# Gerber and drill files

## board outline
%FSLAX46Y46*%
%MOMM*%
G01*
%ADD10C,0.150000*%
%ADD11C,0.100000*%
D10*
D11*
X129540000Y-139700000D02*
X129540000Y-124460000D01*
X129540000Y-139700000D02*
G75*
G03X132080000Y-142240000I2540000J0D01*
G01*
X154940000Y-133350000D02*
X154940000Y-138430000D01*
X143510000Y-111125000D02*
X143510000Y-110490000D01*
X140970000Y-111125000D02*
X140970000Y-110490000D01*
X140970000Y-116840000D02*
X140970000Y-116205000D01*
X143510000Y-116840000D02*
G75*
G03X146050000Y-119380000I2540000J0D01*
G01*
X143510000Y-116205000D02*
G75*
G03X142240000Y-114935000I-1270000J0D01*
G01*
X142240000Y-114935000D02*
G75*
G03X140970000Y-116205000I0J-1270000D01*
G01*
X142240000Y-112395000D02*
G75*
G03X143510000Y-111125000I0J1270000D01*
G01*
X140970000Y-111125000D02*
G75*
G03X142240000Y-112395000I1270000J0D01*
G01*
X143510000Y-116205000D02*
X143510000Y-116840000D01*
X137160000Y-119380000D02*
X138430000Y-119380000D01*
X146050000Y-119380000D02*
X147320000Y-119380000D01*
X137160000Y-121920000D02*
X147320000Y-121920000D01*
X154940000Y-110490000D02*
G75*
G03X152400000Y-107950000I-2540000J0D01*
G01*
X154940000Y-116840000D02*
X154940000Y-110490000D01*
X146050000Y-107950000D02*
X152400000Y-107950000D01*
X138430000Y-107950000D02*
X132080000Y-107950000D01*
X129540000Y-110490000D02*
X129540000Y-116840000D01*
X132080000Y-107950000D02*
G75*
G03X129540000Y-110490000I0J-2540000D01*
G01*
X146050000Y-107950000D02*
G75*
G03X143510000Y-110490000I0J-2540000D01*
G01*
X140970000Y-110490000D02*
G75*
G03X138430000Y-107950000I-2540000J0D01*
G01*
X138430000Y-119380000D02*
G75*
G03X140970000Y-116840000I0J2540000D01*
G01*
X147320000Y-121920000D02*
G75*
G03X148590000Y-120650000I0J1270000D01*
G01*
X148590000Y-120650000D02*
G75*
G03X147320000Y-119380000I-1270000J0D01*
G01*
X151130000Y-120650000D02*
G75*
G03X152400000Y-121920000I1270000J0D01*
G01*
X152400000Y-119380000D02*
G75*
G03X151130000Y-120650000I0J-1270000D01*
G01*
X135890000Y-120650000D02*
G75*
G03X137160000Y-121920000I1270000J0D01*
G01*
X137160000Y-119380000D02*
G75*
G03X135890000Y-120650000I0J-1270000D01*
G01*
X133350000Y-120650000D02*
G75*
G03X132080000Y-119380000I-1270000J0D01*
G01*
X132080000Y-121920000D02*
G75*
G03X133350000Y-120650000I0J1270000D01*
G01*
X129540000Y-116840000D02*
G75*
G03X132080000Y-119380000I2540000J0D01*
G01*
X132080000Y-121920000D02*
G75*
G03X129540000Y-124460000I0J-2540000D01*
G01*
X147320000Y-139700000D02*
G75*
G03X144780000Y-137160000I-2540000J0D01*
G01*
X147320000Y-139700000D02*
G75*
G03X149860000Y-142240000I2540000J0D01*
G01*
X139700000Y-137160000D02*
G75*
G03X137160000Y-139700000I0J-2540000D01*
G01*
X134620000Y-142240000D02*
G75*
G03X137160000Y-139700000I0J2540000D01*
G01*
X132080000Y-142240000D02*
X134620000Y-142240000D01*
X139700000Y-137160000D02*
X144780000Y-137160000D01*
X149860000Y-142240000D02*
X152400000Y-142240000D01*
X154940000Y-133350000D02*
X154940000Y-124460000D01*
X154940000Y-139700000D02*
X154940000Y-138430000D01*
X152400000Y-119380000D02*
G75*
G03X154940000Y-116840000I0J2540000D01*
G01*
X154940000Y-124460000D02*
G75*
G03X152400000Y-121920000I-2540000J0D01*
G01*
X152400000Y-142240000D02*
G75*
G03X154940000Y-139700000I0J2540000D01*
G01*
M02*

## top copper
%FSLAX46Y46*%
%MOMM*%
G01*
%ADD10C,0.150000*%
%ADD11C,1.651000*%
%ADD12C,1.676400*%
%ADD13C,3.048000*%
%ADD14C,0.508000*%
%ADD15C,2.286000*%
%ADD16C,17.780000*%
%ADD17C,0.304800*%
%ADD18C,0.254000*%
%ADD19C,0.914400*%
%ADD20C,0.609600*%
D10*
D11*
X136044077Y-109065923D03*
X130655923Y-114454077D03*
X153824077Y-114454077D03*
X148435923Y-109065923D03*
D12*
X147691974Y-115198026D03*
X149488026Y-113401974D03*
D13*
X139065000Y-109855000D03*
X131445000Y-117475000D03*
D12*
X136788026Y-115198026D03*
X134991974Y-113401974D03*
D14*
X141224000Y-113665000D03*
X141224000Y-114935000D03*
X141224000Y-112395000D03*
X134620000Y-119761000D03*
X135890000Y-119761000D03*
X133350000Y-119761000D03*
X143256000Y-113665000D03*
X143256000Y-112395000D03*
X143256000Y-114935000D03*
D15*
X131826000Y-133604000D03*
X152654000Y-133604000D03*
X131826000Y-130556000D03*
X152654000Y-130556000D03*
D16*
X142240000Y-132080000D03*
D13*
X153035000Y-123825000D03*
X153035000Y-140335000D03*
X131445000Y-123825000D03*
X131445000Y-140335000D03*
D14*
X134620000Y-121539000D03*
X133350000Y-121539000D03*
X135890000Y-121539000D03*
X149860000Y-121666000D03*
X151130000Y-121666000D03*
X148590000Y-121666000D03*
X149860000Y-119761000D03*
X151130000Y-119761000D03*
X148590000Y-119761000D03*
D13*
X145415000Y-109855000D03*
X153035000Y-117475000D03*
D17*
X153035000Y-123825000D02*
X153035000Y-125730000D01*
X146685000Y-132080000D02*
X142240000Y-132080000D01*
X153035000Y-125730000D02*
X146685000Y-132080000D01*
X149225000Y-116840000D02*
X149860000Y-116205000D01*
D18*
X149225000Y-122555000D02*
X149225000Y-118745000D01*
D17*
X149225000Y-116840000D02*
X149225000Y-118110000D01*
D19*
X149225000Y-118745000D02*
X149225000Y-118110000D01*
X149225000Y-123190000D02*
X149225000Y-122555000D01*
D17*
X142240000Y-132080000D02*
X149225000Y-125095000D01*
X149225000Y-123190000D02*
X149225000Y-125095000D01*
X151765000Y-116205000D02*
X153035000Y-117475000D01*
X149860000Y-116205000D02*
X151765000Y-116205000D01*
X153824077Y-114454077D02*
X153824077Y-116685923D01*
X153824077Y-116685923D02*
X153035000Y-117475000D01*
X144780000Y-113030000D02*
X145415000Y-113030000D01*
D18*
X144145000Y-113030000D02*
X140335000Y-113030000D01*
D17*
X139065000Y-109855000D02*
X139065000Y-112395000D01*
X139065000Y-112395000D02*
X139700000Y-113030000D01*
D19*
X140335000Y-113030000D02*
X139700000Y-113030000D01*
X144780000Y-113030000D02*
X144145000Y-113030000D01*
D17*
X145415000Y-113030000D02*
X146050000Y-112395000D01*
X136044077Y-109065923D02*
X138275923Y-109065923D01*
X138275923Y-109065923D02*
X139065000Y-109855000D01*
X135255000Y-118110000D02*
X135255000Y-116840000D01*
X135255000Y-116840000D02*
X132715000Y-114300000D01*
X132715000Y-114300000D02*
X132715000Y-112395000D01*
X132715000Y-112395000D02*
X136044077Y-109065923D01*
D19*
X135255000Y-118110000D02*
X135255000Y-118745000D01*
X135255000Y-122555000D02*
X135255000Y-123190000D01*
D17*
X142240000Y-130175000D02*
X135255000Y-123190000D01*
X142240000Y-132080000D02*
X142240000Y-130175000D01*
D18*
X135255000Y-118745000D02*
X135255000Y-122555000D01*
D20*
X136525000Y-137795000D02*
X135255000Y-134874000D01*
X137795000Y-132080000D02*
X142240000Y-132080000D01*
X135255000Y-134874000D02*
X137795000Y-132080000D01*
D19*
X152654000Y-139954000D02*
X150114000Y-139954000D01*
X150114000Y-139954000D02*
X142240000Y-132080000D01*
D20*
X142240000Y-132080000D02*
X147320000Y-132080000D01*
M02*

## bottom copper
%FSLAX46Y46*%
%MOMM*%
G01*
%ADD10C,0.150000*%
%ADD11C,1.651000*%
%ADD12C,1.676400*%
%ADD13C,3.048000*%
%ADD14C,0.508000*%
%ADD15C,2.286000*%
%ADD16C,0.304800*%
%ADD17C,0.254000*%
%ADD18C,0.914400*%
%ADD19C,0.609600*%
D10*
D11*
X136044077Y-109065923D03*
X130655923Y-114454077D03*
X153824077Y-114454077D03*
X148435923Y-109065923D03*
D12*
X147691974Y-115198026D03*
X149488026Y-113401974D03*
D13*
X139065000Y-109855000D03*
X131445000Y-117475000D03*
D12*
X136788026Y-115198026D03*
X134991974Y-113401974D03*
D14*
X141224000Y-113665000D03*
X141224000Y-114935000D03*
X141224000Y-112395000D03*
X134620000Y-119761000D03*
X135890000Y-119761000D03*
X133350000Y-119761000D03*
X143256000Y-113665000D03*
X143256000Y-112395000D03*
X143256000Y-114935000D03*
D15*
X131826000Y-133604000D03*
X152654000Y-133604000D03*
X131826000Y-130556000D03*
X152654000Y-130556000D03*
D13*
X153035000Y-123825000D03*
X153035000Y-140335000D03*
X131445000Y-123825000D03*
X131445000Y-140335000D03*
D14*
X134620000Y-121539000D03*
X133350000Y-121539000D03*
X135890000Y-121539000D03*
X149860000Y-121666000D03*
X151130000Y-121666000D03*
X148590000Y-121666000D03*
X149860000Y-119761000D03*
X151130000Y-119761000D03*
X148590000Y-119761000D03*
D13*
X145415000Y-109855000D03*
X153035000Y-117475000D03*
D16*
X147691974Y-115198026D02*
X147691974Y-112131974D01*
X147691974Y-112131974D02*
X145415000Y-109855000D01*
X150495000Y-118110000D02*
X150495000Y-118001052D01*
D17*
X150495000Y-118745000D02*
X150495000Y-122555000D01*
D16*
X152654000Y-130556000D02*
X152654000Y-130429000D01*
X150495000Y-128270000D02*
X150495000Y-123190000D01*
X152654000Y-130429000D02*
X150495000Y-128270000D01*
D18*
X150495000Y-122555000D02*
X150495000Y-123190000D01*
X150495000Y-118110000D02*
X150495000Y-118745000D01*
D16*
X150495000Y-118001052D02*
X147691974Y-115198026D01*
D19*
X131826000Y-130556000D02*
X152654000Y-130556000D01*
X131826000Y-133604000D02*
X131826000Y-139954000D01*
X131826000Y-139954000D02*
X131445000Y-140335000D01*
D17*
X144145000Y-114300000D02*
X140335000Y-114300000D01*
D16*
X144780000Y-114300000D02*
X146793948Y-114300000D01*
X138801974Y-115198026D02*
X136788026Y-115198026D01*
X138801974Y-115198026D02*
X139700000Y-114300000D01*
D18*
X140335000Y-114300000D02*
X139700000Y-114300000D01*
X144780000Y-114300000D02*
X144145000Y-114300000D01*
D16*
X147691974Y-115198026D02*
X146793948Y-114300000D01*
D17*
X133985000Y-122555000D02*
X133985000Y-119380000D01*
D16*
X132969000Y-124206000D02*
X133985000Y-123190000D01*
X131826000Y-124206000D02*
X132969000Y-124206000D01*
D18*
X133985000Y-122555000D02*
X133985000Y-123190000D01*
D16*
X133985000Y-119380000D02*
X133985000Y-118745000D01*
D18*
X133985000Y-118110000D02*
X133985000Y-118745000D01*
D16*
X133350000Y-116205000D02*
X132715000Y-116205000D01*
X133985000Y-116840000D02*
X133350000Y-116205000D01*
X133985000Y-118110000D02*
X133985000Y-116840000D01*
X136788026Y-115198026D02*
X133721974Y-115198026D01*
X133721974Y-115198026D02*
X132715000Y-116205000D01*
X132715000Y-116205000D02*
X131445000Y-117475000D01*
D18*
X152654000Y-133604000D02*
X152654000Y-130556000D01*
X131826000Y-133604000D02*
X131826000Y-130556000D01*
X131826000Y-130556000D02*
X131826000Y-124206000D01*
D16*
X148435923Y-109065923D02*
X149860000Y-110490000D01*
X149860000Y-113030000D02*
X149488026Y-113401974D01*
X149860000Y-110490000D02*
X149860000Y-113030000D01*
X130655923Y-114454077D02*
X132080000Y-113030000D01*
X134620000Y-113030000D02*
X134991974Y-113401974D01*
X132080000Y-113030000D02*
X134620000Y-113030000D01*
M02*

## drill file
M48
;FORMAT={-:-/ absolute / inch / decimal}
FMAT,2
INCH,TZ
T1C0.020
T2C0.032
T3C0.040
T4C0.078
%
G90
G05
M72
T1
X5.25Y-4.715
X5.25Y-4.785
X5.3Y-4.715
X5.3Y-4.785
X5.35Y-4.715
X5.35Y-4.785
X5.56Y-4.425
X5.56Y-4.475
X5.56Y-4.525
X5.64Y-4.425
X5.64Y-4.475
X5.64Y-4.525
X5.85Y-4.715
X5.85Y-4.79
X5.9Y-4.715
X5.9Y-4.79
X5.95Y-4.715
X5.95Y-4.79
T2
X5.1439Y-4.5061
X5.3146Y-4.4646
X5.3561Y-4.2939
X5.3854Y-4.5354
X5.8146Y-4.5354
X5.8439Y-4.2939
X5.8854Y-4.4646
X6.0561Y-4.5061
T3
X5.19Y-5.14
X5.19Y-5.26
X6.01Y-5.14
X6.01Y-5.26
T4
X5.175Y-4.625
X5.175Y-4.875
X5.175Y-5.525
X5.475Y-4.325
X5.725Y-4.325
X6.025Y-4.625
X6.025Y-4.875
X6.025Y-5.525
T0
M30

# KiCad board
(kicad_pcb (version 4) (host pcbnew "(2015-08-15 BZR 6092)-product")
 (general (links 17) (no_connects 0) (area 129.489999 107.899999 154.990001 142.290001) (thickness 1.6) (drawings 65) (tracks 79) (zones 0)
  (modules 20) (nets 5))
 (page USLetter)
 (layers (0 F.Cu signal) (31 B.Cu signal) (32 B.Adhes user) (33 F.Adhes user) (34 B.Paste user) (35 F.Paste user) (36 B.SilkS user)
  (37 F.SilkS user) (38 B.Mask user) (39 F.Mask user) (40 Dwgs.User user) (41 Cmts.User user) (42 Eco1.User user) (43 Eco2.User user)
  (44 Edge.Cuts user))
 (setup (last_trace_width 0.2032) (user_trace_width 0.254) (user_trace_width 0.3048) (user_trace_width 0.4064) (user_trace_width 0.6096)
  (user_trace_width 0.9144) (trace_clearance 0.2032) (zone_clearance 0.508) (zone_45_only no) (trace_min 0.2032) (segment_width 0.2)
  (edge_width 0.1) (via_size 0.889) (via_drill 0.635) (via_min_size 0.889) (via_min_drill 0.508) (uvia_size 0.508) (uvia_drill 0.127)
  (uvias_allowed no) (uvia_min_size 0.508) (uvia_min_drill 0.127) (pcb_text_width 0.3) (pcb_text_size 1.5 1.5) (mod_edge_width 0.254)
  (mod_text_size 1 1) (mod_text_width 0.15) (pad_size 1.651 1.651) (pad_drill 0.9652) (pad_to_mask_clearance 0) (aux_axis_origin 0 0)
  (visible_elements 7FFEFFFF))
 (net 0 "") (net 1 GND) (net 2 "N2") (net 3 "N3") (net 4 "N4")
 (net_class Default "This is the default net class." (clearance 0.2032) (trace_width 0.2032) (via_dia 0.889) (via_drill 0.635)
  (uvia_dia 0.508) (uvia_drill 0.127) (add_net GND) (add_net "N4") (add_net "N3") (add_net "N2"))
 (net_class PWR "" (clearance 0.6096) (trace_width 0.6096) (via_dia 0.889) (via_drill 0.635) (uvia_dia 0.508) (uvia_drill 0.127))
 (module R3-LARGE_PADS (layer F.Cu) (at 133.35 111.76 225) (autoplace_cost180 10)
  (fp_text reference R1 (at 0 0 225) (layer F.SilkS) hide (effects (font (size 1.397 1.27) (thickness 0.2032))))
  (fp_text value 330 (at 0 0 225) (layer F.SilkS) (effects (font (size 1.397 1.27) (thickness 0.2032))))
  (pad 1 thru_hole circle (at -3.81 0 225) (size 1.651 1.651) (drill 0.8128) (layers *.Cu *.Mask F.SilkS) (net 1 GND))
  (pad 2 thru_hole circle (at 3.81 0 225) (size 1.651 1.651) (drill 0.8128) (layers *.Cu *.Mask F.SilkS) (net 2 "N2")))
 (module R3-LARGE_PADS (layer F.Cu) (at 151.13 111.76 135) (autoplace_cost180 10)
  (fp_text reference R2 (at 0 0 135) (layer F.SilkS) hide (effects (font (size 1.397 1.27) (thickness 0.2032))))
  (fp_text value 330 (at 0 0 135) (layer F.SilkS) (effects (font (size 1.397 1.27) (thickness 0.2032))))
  (pad 1 thru_hole circle (at -3.81 0 135) (size 1.651 1.651) (drill 0.8128) (layers *.Cu *.Mask F.SilkS) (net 1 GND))
  (pad 2 thru_hole circle (at 3.81 0 135) (size 1.651 1.651) (drill 0.8128) (layers *.Cu *.Mask F.SilkS) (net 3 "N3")))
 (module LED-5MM (layer F.Cu) (at 148.59 114.3 45)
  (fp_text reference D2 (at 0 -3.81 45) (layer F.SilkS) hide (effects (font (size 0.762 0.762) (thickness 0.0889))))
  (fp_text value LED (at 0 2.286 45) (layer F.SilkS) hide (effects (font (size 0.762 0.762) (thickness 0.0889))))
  (pad 1 thru_hole circle (at -1.27 0 45) (size 1.6764 1.6764) (drill 0.8128) (layers *.Cu *.Mask F.SilkS) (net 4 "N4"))
  (pad 2 thru_hole circle (at 1.27 0 45) (size 1.6764 1.6764) (drill 0.8128) (layers *.Cu *.Mask F.SilkS) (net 3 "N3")))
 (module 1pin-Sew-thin (layer F.Cu) (at 139.065 109.855 270)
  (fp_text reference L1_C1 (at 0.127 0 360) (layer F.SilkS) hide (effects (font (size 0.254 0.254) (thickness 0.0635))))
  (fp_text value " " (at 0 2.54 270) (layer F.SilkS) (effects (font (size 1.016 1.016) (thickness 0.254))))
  (pad 1 thru_hole circle (at 0 0 270) (size 3.048 3.048) (drill 1.984375) (layers *.Cu *.Mask F.SilkS) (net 1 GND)))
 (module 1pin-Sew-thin (layer F.Cu) (at 131.445 117.475 270)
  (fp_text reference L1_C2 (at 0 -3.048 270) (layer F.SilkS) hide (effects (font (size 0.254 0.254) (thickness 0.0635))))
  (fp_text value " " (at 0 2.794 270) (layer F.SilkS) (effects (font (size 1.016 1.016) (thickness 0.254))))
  (pad 1 thru_hole circle (at 0 0 270) (size 3.048 3.048) (drill 1.984375) (layers *.Cu *.Mask F.SilkS) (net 4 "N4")))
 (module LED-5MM (layer F.Cu) (at 135.89 114.3 135)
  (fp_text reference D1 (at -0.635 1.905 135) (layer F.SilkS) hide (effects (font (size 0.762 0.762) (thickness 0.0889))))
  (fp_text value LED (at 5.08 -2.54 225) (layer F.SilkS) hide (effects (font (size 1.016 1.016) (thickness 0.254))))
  (pad 1 thru_hole circle (at -1.27 0 135) (size 1.6764 1.6764) (drill 0.8128) (layers *.Cu *.Mask F.SilkS) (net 4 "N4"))
  (pad 2 thru_hole circle (at 1.27 0 135) (size 1.6764 1.6764) (drill 0.8128) (layers *.Cu *.Mask F.SilkS) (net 2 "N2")))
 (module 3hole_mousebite (layer F.Cu) (at 141.605 113.665 90)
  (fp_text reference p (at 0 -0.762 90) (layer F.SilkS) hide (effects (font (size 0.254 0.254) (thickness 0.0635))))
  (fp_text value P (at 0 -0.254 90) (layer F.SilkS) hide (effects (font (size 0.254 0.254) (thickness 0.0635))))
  (pad "" thru_hole circle (at 0 -0.381 90) (size 0.508 0.508) (drill 0.508) (layers *.Cu *.Mask F.SilkS))
  (pad 1 thru_hole circle (at -1.27 -0.381 90) (size 0.508 0.508) (drill 0.508) (layers *.Cu *.Mask F.SilkS))
  (pad 2 thru_hole circle (at 1.27 -0.381 90) (size 0.508 0.508) (drill 0.508) (layers *.Cu *.Mask F.SilkS)))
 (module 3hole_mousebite (layer F.Cu) (at 134.62 119.38 180)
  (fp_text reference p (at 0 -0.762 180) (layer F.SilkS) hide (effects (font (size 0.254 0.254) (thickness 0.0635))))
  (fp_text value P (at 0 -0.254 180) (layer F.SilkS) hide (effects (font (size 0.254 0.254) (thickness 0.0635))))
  (pad "" thru_hole circle (at 0 -0.381 180) (size 0.508 0.508) (drill 0.508) (layers *.Cu *.Mask F.SilkS))
  (pad 1 thru_hole circle (at -1.27 -0.381 180) (size 0.508 0.508) (drill 0.508) (layers *.Cu *.Mask F.SilkS))
  (pad 2 thru_hole circle (at 1.27 -0.381 180) (size 0.508 0.508) (drill 0.508) (layers *.Cu *.Mask F.SilkS)))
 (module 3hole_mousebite (layer F.Cu) (at 142.875 113.665 270)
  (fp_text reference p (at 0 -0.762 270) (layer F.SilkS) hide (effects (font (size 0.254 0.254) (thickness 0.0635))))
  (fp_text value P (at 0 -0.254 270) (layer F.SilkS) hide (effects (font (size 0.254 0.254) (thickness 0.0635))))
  (pad "" thru_hole circle (at 0 -0.381 270) (size 0.508 0.508) (drill 0.508) (layers *.Cu *.Mask F.SilkS))
  (pad 1 thru_hole circle (at -1.27 -0.381 270) (size 0.508 0.508) (drill 0.508) (layers *.Cu *.Mask F.SilkS))
  (pad 2 thru_hole circle (at 1.27 -0.381 270) (size 0.508 0.508) (drill 0.508) (layers *.Cu *.Mask F.SilkS)))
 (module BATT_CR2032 (layer F.Cu) (at 142.24 132.08)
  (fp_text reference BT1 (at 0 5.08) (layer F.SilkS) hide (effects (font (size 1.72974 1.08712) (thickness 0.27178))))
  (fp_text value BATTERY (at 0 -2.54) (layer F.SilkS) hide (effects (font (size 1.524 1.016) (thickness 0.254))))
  (pad 1 thru_hole circle (at -10.414 1.524) (size 2.286 2.286) (drill 1.016) (layers *.Cu *.Mask F.SilkS) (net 4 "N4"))
  (pad 1 thru_hole circle (at 10.414 1.524) (size 2.286 2.286) (drill 1.016) (layers *.Cu *.Mask F.SilkS) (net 4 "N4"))
  (pad 1 thru_hole circle (at -10.414 -1.524) (size 2.286 2.286) (drill 1.016) (layers *.Cu *.Mask F.SilkS) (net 4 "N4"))
  (pad 1 thru_hole circle (at 10.414 -1.524) (size 2.286 2.286) (drill 1.016) (layers *.Cu *.Mask F.SilkS) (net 4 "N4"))
  (pad 2 smd circle (at 0 0) (size 17.78 17.78) (layers F.Cu F.Paste F.Mask) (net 1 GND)))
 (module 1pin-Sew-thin (layer F.Cu) (at 153.035 123.825)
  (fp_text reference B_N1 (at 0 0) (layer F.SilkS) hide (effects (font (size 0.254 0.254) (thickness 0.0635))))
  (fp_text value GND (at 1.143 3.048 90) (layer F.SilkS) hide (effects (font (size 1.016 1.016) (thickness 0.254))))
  (pad 1 thru_hole circle (at 0 0) (size 3.048 3.048) (drill 1.984375) (layers *.Cu *.Mask F.SilkS) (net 1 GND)))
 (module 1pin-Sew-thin (layer F.Cu) (at 153.035 140.335)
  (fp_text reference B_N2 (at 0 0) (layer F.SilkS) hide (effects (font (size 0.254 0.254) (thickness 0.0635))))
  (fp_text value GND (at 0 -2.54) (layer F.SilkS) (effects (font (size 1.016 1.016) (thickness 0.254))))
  (pad 1 thru_hole circle (at 0 0) (size 3.048 3.048) (drill 1.984375) (layers *.Cu *.Mask F.SilkS) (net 1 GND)))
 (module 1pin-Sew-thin (layer F.Cu) (at 131.445 123.825)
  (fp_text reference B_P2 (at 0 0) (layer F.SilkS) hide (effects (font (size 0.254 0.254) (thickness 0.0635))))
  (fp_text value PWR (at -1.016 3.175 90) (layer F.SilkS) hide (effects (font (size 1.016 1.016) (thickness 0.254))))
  (pad 1 thru_hole circle (at 0 0) (size 3.048 3.048) (drill 1.984375) (layers *.Cu *.Mask F.SilkS) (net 4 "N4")))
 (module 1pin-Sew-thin (layer F.Cu) (at 131.445 140.335)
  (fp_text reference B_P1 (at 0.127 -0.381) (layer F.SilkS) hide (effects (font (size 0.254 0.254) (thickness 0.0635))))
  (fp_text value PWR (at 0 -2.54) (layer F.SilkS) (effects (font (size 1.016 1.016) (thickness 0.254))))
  (pad 1 thru_hole circle (at 0 0) (size 3.048 3.048) (drill 1.984375) (layers *.Cu *.Mask F.SilkS) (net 4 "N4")))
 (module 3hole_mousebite (layer F.Cu) (at 134.62 121.92)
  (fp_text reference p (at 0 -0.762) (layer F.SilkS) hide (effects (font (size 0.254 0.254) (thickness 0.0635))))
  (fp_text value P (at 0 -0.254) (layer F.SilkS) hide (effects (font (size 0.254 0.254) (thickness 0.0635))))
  (pad "" thru_hole circle (at 0 -0.381) (size 0.508 0.508) (drill 0.508) (layers *.Cu *.Mask F.SilkS))
  (pad 1 thru_hole circle (at -1.27 -0.381) (size 0.508 0.508) (drill 0.508) (layers *.Cu *.Mask F.SilkS))
  (pad 2 thru_hole circle (at 1.27 -0.381) (size 0.508 0.508) (drill 0.508) (layers *.Cu *.Mask F.SilkS)))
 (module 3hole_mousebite (layer F.Cu) (at 149.86 121.285 180)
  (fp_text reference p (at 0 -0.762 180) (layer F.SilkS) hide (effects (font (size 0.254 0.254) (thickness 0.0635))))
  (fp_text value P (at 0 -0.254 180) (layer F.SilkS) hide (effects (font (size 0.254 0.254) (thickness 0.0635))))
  (pad "" thru_hole circle (at 0 -0.381 180) (size 0.508 0.508) (drill 0.508) (layers *.Cu *.Mask F.SilkS))
  (pad 1 thru_hole circle (at -1.27 -0.381 180) (size 0.508 0.508) (drill 0.508) (layers *.Cu *.Mask F.SilkS))
  (pad 2 thru_hole circle (at 1.27 -0.381 180) (size 0.508 0.508) (drill 0.508) (layers *.Cu *.Mask F.SilkS)))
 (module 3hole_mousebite (layer F.Cu) (at 149.86 119.38 180)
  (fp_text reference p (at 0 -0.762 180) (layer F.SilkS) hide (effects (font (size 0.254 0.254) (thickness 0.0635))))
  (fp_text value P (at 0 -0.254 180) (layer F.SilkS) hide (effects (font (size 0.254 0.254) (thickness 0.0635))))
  (pad "" thru_hole circle (at 0 -0.381 180) (size 0.508 0.508) (drill 0.508) (layers *.Cu *.Mask F.SilkS))
  (pad 1 thru_hole circle (at -1.27 -0.381 180) (size 0.508 0.508) (drill 0.508) (layers *.Cu *.Mask F.SilkS))
  (pad 2 thru_hole circle (at 1.27 -0.381 180) (size 0.508 0.508) (drill 0.508) (layers *.Cu *.Mask F.SilkS)))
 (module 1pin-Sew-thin (layer F.Cu) (at 145.415 109.855)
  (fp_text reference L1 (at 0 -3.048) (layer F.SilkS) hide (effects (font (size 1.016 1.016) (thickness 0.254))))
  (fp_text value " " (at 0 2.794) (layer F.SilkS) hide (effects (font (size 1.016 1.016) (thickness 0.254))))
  (pad 1 thru_hole circle (at 0 0) (size 3.048 3.048) (drill 1.984375) (layers *.Cu *.Mask F.SilkS) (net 4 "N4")))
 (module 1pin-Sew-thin (layer F.Cu) (at 153.035 117.475)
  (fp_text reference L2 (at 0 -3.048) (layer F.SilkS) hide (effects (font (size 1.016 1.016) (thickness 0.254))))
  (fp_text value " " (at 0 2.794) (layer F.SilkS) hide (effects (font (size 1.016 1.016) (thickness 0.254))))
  (pad 1 thru_hole circle (at 0 0) (size 3.048 3.048) (drill 1.984375) (layers *.Cu *.Mask F.SilkS) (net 1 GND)))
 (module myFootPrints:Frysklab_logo (layer F.Cu) (at 142 132)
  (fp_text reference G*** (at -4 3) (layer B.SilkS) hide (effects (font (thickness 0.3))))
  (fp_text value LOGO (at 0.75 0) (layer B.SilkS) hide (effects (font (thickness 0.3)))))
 (gr_line (start 129.54 139.7) (end 129.54 124.46) (angle 90) (layer Edge.Cuts) (width 0.1))
 (gr_arc (start 132.08 139.7) (end 132.08 142.24) (angle 90) (layer Edge.Cuts) (width 0.1))
 (gr_line (start 154.94 133.35) (end 154.94 138.43) (angle 90) (layer Edge.Cuts) (width 0.1))
 (gr_line (start 143.51 111.125) (end 143.51 110.49) (angle 90) (layer Edge.Cuts) (width 0.1))
 (gr_line (start 140.97 111.125) (end 140.97 110.49) (angle 90) (layer Edge.Cuts) (width 0.1))
 (gr_line (start 140.97 116.84) (end 140.97 116.205) (angle 90) (layer Edge.Cuts) (width 0.1))
 (gr_arc (start 146.05 116.84) (end 146.05 119.38) (angle 90) (layer Edge.Cuts) (width 0.1))
 (gr_arc (start 142.24 116.205) (end 142.24 114.935) (angle 90) (layer Edge.Cuts) (width 0.1))
 (gr_arc (start 142.24 116.205) (end 140.97 116.205) (angle 90) (layer Edge.Cuts) (width 0.1))
 (gr_arc (start 142.24 111.125) (end 143.51 111.125) (angle 90) (layer Edge.Cuts) (width 0.1))
 (gr_arc (start 142.24 111.125) (end 142.24 112.395) (angle 90) (layer Edge.Cuts) (width 0.1))
 (gr_line (start 143.51 116.205) (end 143.51 116.84) (angle 90) (layer Edge.Cuts) (width 0.1))
 (gr_line (start 137.16 119.38) (end 138.43 119.38) (angle 90) (layer Edge.Cuts) (width 0.1))
 (gr_line (start 146.05 119.38) (end 147.32 119.38) (angle 90) (layer Edge.Cuts) (width 0.1))
 (gr_line (start 137.16 121.92) (end 147.32 121.92) (angle 90) (layer Edge.Cuts) (width 0.1))
 (gr_arc (start 152.4 110.49) (end 152.4 107.95) (angle 90) (layer Edge.Cuts) (width 0.1))
 (gr_line (start 154.94 116.84) (end 154.94 110.49) (angle 90) (layer Edge.Cuts) (width 0.1))
 (gr_line (start 146.05 107.95) (end 152.4 107.95) (angle 90) (layer Edge.Cuts) (width 0.1))
 (gr_line (start 138.43 107.95) (end 132.08 107.95) (angle 90) (layer Edge.Cuts) (width 0.1))
 (gr_line (start 129.54 110.49) (end 129.54 116.84) (angle 90) (layer Edge.Cuts) (width 0.1))
 (gr_arc (start 132.08 110.49) (end 129.54 110.49) (angle 90) (layer Edge.Cuts) (width 0.1))
 (gr_arc (start 146.05 110.49) (end 143.51 110.49) (angle 90) (layer Edge.Cuts) (width 0.1))
 (gr_arc (start 138.43 110.49) (end 138.43 107.95) (angle 90) (layer Edge.Cuts) (width 0.1))
 (gr_arc (start 138.43 116.84) (end 140.97 116.84) (angle 90) (layer Edge.Cuts) (width 0.1))
 (gr_arc (start 147.32 120.65) (end 148.59 120.65) (angle 90) (layer Edge.Cuts) (width 0.1))
 (gr_arc (start 147.32 120.65) (end 147.32 119.38) (angle 90) (layer Edge.Cuts) (width 0.1))
 (gr_arc (start 152.4 120.65) (end 152.4 121.92) (angle 90) (layer Edge.Cuts) (width 0.1))
 (gr_arc (start 152.4 120.65) (end 151.13 120.65) (angle 90) (layer Edge.Cuts) (width 0.1))
 (gr_arc (start 137.16 120.65) (end 137.16 121.92) (angle 90) (layer Edge.Cuts) (width 0.1))
 (gr_arc (start 137.16 120.65) (end 135.89 120.65) (angle 90) (layer Edge.Cuts) (width 0.1))
 (gr_arc (start 132.08 120.65) (end 132.08 119.38) (angle 90) (layer Edge.Cuts) (width 0.1))
 (gr_arc (start 132.08 120.65) (end 133.35 120.65) (angle 90) (layer Edge.Cuts) (width 0.1))
 (gr_arc (start 132.08 116.84) (end 132.08 119.38) (angle 90) (layer Edge.Cuts) (width 0.1))
 (gr_arc (start 132.08 124.46) (end 129.54 124.46) (angle 90) (layer Edge.Cuts) (width 0.1))
 (gr_arc (start 144.78 139.7) (end 144.78 137.16) (angle 90) (layer Edge.Cuts) (width 0.1))
 (gr_arc (start 149.86 139.7) (end 149.86 142.24) (angle 90) (layer Edge.Cuts) (width 0.1))
 (gr_arc (start 139.7 139.7) (end 137.16 139.7) (angle 90) (layer Edge.Cuts) (width 0.1))
 (gr_arc (start 134.62 139.7) (end 137.16 139.7) (angle 90) (layer Edge.Cuts) (width 0.1))
 (gr_line (start 132.08 142.24) (end 134.62 142.24) (angle 90) (layer Edge.Cuts) (width 0.1))
 (gr_line (start 139.7 137.16) (end 144.78 137.16) (angle 90) (layer Edge.Cuts) (width 0.1))
 (gr_line (start 149.86 142.24) (end 152.4 142.24) (angle 90) (layer Edge.Cuts) (width 0.1))
 (gr_line (start 154.94 133.35) (end 154.94 124.46) (angle 90) (layer Edge.Cuts) (width 0.1))
 (gr_line (start 154.94 139.7) (end 154.94 138.43) (angle 90) (layer Edge.Cuts) (width 0.1))
 (gr_arc (start 152.4 116.84) (end 154.94 116.84) (angle 90) (layer Edge.Cuts) (width 0.1))
 (gr_arc (start 152.4 124.46) (end 152.4 121.92) (angle 90) (layer Edge.Cuts) (width 0.1))
 (gr_arc (start 152.4 139.7) (end 154.94 139.7) (angle 90) (layer Edge.Cuts) (width 0.1))
 (segment (start 153.035 123.825) (end 153.035 125.73) (width 0.3048) (layer F.Cu) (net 1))
 (segment (start 146.685 132.08) (end 142.24 132.08) (width 0.3048) (layer F.Cu) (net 1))
 (segment (start 153.035 125.73) (end 146.685 132.08) (width 0.3048) (layer F.Cu) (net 1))
 (segment (start 149.225 116.84) (end 149.86 116.205) (width 0.3048) (layer F.Cu) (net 1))
 (segment (start 149.225 122.555) (end 149.225 118.745) (width 0.254) (layer F.Cu) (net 1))
 (segment (start 149.225 116.84) (end 149.225 118.11) (width 0.3048) (layer F.Cu) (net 1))
 (segment (start 149.225 118.745) (end 149.225 118.11) (width 0.9144) (layer F.Cu) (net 1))
 (segment (start 149.225 123.19) (end 149.225 122.555) (width 0.9144) (layer F.Cu) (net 1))
 (segment (start 142.24 132.08) (end 149.225 125.095) (width 0.3048) (layer F.Cu) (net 1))
 (segment (start 149.225 123.19) (end 149.225 125.095) (width 0.3048) (layer F.Cu) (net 1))
 (segment (start 151.765 116.205) (end 153.035 117.475) (width 0.3048) (layer F.Cu) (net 1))
 (segment (start 149.86 116.205) (end 151.765 116.205) (width 0.3048) (layer F.Cu) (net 1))
 (segment (start 153.824077 114.454077) (end 153.824077 116.685923) (width 0.3048) (layer F.Cu) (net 1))
 (segment (start 153.824077 116.685923) (end 153.035 117.475) (width 0.3048) (layer F.Cu) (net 1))
 (segment (start 144.78 113.03) (end 145.415 113.03) (width 0.3048) (layer F.Cu) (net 1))
 (segment (start 144.145 113.03) (end 140.335 113.03) (width 0.254) (layer F.Cu) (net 1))
 (segment (start 139.065 109.855) (end 139.065 112.395) (width 0.3048) (layer F.Cu) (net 1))
 (segment (start 139.065 112.395) (end 139.7 113.03) (width 0.3048) (layer F.Cu) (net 1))
 (segment (start 140.335 113.03) (end 139.7 113.03) (width 0.9144) (layer F.Cu) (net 1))
 (segment (start 144.78 113.03) (end 144.145 113.03) (width 0.9144) (layer F.Cu) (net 1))
 (segment (start 145.415 113.03) (end 146.05 112.395) (width 0.3048) (layer F.Cu) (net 1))
 (segment (start 136.044077 109.065923) (end 138.275923 109.065923) (width 0.3048) (layer F.Cu) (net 1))
 (segment (start 138.275923 109.065923) (end 139.065 109.855) (width 0.3048) (layer F.Cu) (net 1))
 (segment (start 135.255 118.11) (end 135.255 116.84) (width 0.3048) (layer F.Cu) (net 1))
 (segment (start 135.255 116.84) (end 132.715 114.3) (width 0.3048) (layer F.Cu) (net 1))
 (segment (start 132.715 114.3) (end 132.715 112.395) (width 0.3048) (layer F.Cu) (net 1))
 (segment (start 132.715 112.395) (end 136.044077 109.065923) (width 0.3048) (layer F.Cu) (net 1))
 (segment (start 135.255 118.11) (end 135.255 118.745) (width 0.9144) (layer F.Cu) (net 1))
 (segment (start 135.255 122.555) (end 135.255 123.19) (width 0.9144) (layer F.Cu) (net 1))
 (segment (start 142.24 130.175) (end 135.255 123.19) (width 0.3048) (layer F.Cu) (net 1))
 (segment (start 142.24 132.08) (end 142.24 130.175) (width 0.3048) (layer F.Cu) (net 1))
 (segment (start 135.255 118.745) (end 135.255 122.555) (width 0.254) (layer F.Cu) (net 1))
 (segment (start 136.525 137.795) (end 135.255 134.874) (width 0.6096) (layer F.Cu) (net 1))
 (segment (start 137.795 132.08) (end 142.24 132.08) (width 0.6096) (layer F.Cu) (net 1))
 (segment (start 135.255 134.874) (end 137.795 132.08) (width 0.6096) (layer F.Cu) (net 1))
 (segment (start 152.654 139.954) (end 150.114 139.954) (width 0.9144) (layer F.Cu) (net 1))
 (segment (start 150.114 139.954) (end 142.24 132.08) (width 0.9144) (layer F.Cu) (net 1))
 (segment (start 142.24 132.08) (end 147.32 132.08) (width 0.6096) (layer F.Cu) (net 1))
 (segment (start 147.691974 115.198026) (end 147.691974 112.131974) (width 0.3048) (layer B.Cu) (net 4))
 (segment (start 147.691974 112.131974) (end 145.415 109.855) (width 0.3048) (layer B.Cu) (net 4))
 (segment (start 150.495 118.11) (end 150.495 118.001052) (width 0.3048) (layer B.Cu) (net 4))
 (segment (start 150.495 118.745) (end 150.495 122.555) (width 0.254) (layer B.Cu) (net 4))
 (segment (start 152.654 130.556) (end 152.654 130.429) (width 0.3048) (layer B.Cu) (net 4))
 (segment (start 150.495 128.27) (end 150.495 123.19) (width 0.3048) (layer B.Cu) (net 4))
 (segment (start 152.654 130.429) (end 150.495 128.27) (width 0.3048) (layer B.Cu) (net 4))
 (segment (start 150.495 122.555) (end 150.495 123.19) (width 0.9144) (layer B.Cu) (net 4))
 (segment (start 150.495 118.11) (end 150.495 118.745) (width 0.9144) (layer B.Cu) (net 4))
 (segment (start 150.495 118.001052) (end 147.691974 115.198026) (width 0.3048) (layer B.Cu) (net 4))
 (segment (start 131.826 130.556) (end 152.654 130.556) (width 0.6096) (layer B.Cu) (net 4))
 (segment (start 131.826 133.604) (end 131.826 139.954) (width 0.6096) (layer B.Cu) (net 4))
 (segment (start 131.826 139.954) (end 131.445 140.335) (width 0.6096) (layer B.Cu) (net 4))
 (segment (start 144.145 114.3) (end 140.335 114.3) (width 0.254) (layer B.Cu) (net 4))
 (segment (start 144.78 114.3) (end 146.793948 114.3) (width 0.3048) (layer B.Cu) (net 4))
 (segment (start 138.801974 115.198026) (end 136.788026 115.198026) (width 0.3048) (layer B.Cu) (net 4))
 (segment (start 138.801974 115.198026) (end 139.7 114.3) (width 0.3048) (layer B.Cu) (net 4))
 (segment (start 140.335 114.3) (end 139.7 114.3) (width 0.9144) (layer B.Cu) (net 4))
 (segment (start 144.78 114.3) (end 144.145 114.3) (width 0.9144) (layer B.Cu) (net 4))
 (segment (start 147.691974 115.198026) (end 146.793948 114.3) (width 0.3048) (layer B.Cu) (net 4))
 (segment (start 133.985 122.555) (end 133.985 119.38) (width 0.254) (layer B.Cu) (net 4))
 (segment (start 132.969 124.206) (end 133.985 123.19) (width 0.3048) (layer B.Cu) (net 4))
 (segment (start 131.826 124.206) (end 132.969 124.206) (width 0.3048) (layer B.Cu) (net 4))
 (segment (start 133.985 122.555) (end 133.985 123.19) (width 0.9144) (layer B.Cu) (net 4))
 (segment (start 133.985 119.38) (end 133.985 118.745) (width 0.3048) (layer B.Cu) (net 4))
 (segment (start 133.985 118.11) (end 133.985 118.745) (width 0.9144) (layer B.Cu) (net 4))
 (segment (start 133.35 116.205) (end 132.715 116.205) (width 0.3048) (layer B.Cu) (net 4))
 (segment (start 133.985 116.84) (end 133.35 116.205) (width 0.3048) (layer B.Cu) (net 4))
 (segment (start 133.985 118.11) (end 133.985 116.84) (width 0.3048) (layer B.Cu) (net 4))
 (segment (start 136.788026 115.198026) (end 133.721974 115.198026) (width 0.3048) (layer B.Cu) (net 4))
 (segment (start 133.721974 115.198026) (end 132.715 116.205) (width 0.3048) (layer B.Cu) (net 4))
 (segment (start 132.715 116.205) (end 131.445 117.475) (width 0.3048) (layer B.Cu) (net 4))
 (segment (start 152.654 133.604) (end 152.654 130.556) (width 0.9144) (layer B.Cu) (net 4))
 (segment (start 131.826 133.604) (end 131.826 130.556) (width 0.9144) (layer B.Cu) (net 4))
 (segment (start 131.826 130.556) (end 131.826 124.206) (width 0.9144) (layer B.Cu) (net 4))
 (segment (start 148.435923 109.065923) (end 149.86 110.49) (width 0.3048) (layer B.Cu) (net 3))
 (segment (start 149.86 113.03) (end 149.488026 113.401974) (width 0.3048) (layer B.Cu) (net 3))
 (segment (start 149.86 110.49) (end 149.86 113.03) (width 0.3048) (layer B.Cu) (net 3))
 (segment (start 130.655923 114.454077) (end 132.08 113.03) (width 0.3048) (layer B.Cu) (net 2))
 (segment (start 134.62 113.03) (end 134.991974 113.401974) (width 0.3048) (layer B.Cu) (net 2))
 (segment (start 132.08 113.03) (end 134.62 113.03) (width 0.3048) (layer B.Cu) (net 2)))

